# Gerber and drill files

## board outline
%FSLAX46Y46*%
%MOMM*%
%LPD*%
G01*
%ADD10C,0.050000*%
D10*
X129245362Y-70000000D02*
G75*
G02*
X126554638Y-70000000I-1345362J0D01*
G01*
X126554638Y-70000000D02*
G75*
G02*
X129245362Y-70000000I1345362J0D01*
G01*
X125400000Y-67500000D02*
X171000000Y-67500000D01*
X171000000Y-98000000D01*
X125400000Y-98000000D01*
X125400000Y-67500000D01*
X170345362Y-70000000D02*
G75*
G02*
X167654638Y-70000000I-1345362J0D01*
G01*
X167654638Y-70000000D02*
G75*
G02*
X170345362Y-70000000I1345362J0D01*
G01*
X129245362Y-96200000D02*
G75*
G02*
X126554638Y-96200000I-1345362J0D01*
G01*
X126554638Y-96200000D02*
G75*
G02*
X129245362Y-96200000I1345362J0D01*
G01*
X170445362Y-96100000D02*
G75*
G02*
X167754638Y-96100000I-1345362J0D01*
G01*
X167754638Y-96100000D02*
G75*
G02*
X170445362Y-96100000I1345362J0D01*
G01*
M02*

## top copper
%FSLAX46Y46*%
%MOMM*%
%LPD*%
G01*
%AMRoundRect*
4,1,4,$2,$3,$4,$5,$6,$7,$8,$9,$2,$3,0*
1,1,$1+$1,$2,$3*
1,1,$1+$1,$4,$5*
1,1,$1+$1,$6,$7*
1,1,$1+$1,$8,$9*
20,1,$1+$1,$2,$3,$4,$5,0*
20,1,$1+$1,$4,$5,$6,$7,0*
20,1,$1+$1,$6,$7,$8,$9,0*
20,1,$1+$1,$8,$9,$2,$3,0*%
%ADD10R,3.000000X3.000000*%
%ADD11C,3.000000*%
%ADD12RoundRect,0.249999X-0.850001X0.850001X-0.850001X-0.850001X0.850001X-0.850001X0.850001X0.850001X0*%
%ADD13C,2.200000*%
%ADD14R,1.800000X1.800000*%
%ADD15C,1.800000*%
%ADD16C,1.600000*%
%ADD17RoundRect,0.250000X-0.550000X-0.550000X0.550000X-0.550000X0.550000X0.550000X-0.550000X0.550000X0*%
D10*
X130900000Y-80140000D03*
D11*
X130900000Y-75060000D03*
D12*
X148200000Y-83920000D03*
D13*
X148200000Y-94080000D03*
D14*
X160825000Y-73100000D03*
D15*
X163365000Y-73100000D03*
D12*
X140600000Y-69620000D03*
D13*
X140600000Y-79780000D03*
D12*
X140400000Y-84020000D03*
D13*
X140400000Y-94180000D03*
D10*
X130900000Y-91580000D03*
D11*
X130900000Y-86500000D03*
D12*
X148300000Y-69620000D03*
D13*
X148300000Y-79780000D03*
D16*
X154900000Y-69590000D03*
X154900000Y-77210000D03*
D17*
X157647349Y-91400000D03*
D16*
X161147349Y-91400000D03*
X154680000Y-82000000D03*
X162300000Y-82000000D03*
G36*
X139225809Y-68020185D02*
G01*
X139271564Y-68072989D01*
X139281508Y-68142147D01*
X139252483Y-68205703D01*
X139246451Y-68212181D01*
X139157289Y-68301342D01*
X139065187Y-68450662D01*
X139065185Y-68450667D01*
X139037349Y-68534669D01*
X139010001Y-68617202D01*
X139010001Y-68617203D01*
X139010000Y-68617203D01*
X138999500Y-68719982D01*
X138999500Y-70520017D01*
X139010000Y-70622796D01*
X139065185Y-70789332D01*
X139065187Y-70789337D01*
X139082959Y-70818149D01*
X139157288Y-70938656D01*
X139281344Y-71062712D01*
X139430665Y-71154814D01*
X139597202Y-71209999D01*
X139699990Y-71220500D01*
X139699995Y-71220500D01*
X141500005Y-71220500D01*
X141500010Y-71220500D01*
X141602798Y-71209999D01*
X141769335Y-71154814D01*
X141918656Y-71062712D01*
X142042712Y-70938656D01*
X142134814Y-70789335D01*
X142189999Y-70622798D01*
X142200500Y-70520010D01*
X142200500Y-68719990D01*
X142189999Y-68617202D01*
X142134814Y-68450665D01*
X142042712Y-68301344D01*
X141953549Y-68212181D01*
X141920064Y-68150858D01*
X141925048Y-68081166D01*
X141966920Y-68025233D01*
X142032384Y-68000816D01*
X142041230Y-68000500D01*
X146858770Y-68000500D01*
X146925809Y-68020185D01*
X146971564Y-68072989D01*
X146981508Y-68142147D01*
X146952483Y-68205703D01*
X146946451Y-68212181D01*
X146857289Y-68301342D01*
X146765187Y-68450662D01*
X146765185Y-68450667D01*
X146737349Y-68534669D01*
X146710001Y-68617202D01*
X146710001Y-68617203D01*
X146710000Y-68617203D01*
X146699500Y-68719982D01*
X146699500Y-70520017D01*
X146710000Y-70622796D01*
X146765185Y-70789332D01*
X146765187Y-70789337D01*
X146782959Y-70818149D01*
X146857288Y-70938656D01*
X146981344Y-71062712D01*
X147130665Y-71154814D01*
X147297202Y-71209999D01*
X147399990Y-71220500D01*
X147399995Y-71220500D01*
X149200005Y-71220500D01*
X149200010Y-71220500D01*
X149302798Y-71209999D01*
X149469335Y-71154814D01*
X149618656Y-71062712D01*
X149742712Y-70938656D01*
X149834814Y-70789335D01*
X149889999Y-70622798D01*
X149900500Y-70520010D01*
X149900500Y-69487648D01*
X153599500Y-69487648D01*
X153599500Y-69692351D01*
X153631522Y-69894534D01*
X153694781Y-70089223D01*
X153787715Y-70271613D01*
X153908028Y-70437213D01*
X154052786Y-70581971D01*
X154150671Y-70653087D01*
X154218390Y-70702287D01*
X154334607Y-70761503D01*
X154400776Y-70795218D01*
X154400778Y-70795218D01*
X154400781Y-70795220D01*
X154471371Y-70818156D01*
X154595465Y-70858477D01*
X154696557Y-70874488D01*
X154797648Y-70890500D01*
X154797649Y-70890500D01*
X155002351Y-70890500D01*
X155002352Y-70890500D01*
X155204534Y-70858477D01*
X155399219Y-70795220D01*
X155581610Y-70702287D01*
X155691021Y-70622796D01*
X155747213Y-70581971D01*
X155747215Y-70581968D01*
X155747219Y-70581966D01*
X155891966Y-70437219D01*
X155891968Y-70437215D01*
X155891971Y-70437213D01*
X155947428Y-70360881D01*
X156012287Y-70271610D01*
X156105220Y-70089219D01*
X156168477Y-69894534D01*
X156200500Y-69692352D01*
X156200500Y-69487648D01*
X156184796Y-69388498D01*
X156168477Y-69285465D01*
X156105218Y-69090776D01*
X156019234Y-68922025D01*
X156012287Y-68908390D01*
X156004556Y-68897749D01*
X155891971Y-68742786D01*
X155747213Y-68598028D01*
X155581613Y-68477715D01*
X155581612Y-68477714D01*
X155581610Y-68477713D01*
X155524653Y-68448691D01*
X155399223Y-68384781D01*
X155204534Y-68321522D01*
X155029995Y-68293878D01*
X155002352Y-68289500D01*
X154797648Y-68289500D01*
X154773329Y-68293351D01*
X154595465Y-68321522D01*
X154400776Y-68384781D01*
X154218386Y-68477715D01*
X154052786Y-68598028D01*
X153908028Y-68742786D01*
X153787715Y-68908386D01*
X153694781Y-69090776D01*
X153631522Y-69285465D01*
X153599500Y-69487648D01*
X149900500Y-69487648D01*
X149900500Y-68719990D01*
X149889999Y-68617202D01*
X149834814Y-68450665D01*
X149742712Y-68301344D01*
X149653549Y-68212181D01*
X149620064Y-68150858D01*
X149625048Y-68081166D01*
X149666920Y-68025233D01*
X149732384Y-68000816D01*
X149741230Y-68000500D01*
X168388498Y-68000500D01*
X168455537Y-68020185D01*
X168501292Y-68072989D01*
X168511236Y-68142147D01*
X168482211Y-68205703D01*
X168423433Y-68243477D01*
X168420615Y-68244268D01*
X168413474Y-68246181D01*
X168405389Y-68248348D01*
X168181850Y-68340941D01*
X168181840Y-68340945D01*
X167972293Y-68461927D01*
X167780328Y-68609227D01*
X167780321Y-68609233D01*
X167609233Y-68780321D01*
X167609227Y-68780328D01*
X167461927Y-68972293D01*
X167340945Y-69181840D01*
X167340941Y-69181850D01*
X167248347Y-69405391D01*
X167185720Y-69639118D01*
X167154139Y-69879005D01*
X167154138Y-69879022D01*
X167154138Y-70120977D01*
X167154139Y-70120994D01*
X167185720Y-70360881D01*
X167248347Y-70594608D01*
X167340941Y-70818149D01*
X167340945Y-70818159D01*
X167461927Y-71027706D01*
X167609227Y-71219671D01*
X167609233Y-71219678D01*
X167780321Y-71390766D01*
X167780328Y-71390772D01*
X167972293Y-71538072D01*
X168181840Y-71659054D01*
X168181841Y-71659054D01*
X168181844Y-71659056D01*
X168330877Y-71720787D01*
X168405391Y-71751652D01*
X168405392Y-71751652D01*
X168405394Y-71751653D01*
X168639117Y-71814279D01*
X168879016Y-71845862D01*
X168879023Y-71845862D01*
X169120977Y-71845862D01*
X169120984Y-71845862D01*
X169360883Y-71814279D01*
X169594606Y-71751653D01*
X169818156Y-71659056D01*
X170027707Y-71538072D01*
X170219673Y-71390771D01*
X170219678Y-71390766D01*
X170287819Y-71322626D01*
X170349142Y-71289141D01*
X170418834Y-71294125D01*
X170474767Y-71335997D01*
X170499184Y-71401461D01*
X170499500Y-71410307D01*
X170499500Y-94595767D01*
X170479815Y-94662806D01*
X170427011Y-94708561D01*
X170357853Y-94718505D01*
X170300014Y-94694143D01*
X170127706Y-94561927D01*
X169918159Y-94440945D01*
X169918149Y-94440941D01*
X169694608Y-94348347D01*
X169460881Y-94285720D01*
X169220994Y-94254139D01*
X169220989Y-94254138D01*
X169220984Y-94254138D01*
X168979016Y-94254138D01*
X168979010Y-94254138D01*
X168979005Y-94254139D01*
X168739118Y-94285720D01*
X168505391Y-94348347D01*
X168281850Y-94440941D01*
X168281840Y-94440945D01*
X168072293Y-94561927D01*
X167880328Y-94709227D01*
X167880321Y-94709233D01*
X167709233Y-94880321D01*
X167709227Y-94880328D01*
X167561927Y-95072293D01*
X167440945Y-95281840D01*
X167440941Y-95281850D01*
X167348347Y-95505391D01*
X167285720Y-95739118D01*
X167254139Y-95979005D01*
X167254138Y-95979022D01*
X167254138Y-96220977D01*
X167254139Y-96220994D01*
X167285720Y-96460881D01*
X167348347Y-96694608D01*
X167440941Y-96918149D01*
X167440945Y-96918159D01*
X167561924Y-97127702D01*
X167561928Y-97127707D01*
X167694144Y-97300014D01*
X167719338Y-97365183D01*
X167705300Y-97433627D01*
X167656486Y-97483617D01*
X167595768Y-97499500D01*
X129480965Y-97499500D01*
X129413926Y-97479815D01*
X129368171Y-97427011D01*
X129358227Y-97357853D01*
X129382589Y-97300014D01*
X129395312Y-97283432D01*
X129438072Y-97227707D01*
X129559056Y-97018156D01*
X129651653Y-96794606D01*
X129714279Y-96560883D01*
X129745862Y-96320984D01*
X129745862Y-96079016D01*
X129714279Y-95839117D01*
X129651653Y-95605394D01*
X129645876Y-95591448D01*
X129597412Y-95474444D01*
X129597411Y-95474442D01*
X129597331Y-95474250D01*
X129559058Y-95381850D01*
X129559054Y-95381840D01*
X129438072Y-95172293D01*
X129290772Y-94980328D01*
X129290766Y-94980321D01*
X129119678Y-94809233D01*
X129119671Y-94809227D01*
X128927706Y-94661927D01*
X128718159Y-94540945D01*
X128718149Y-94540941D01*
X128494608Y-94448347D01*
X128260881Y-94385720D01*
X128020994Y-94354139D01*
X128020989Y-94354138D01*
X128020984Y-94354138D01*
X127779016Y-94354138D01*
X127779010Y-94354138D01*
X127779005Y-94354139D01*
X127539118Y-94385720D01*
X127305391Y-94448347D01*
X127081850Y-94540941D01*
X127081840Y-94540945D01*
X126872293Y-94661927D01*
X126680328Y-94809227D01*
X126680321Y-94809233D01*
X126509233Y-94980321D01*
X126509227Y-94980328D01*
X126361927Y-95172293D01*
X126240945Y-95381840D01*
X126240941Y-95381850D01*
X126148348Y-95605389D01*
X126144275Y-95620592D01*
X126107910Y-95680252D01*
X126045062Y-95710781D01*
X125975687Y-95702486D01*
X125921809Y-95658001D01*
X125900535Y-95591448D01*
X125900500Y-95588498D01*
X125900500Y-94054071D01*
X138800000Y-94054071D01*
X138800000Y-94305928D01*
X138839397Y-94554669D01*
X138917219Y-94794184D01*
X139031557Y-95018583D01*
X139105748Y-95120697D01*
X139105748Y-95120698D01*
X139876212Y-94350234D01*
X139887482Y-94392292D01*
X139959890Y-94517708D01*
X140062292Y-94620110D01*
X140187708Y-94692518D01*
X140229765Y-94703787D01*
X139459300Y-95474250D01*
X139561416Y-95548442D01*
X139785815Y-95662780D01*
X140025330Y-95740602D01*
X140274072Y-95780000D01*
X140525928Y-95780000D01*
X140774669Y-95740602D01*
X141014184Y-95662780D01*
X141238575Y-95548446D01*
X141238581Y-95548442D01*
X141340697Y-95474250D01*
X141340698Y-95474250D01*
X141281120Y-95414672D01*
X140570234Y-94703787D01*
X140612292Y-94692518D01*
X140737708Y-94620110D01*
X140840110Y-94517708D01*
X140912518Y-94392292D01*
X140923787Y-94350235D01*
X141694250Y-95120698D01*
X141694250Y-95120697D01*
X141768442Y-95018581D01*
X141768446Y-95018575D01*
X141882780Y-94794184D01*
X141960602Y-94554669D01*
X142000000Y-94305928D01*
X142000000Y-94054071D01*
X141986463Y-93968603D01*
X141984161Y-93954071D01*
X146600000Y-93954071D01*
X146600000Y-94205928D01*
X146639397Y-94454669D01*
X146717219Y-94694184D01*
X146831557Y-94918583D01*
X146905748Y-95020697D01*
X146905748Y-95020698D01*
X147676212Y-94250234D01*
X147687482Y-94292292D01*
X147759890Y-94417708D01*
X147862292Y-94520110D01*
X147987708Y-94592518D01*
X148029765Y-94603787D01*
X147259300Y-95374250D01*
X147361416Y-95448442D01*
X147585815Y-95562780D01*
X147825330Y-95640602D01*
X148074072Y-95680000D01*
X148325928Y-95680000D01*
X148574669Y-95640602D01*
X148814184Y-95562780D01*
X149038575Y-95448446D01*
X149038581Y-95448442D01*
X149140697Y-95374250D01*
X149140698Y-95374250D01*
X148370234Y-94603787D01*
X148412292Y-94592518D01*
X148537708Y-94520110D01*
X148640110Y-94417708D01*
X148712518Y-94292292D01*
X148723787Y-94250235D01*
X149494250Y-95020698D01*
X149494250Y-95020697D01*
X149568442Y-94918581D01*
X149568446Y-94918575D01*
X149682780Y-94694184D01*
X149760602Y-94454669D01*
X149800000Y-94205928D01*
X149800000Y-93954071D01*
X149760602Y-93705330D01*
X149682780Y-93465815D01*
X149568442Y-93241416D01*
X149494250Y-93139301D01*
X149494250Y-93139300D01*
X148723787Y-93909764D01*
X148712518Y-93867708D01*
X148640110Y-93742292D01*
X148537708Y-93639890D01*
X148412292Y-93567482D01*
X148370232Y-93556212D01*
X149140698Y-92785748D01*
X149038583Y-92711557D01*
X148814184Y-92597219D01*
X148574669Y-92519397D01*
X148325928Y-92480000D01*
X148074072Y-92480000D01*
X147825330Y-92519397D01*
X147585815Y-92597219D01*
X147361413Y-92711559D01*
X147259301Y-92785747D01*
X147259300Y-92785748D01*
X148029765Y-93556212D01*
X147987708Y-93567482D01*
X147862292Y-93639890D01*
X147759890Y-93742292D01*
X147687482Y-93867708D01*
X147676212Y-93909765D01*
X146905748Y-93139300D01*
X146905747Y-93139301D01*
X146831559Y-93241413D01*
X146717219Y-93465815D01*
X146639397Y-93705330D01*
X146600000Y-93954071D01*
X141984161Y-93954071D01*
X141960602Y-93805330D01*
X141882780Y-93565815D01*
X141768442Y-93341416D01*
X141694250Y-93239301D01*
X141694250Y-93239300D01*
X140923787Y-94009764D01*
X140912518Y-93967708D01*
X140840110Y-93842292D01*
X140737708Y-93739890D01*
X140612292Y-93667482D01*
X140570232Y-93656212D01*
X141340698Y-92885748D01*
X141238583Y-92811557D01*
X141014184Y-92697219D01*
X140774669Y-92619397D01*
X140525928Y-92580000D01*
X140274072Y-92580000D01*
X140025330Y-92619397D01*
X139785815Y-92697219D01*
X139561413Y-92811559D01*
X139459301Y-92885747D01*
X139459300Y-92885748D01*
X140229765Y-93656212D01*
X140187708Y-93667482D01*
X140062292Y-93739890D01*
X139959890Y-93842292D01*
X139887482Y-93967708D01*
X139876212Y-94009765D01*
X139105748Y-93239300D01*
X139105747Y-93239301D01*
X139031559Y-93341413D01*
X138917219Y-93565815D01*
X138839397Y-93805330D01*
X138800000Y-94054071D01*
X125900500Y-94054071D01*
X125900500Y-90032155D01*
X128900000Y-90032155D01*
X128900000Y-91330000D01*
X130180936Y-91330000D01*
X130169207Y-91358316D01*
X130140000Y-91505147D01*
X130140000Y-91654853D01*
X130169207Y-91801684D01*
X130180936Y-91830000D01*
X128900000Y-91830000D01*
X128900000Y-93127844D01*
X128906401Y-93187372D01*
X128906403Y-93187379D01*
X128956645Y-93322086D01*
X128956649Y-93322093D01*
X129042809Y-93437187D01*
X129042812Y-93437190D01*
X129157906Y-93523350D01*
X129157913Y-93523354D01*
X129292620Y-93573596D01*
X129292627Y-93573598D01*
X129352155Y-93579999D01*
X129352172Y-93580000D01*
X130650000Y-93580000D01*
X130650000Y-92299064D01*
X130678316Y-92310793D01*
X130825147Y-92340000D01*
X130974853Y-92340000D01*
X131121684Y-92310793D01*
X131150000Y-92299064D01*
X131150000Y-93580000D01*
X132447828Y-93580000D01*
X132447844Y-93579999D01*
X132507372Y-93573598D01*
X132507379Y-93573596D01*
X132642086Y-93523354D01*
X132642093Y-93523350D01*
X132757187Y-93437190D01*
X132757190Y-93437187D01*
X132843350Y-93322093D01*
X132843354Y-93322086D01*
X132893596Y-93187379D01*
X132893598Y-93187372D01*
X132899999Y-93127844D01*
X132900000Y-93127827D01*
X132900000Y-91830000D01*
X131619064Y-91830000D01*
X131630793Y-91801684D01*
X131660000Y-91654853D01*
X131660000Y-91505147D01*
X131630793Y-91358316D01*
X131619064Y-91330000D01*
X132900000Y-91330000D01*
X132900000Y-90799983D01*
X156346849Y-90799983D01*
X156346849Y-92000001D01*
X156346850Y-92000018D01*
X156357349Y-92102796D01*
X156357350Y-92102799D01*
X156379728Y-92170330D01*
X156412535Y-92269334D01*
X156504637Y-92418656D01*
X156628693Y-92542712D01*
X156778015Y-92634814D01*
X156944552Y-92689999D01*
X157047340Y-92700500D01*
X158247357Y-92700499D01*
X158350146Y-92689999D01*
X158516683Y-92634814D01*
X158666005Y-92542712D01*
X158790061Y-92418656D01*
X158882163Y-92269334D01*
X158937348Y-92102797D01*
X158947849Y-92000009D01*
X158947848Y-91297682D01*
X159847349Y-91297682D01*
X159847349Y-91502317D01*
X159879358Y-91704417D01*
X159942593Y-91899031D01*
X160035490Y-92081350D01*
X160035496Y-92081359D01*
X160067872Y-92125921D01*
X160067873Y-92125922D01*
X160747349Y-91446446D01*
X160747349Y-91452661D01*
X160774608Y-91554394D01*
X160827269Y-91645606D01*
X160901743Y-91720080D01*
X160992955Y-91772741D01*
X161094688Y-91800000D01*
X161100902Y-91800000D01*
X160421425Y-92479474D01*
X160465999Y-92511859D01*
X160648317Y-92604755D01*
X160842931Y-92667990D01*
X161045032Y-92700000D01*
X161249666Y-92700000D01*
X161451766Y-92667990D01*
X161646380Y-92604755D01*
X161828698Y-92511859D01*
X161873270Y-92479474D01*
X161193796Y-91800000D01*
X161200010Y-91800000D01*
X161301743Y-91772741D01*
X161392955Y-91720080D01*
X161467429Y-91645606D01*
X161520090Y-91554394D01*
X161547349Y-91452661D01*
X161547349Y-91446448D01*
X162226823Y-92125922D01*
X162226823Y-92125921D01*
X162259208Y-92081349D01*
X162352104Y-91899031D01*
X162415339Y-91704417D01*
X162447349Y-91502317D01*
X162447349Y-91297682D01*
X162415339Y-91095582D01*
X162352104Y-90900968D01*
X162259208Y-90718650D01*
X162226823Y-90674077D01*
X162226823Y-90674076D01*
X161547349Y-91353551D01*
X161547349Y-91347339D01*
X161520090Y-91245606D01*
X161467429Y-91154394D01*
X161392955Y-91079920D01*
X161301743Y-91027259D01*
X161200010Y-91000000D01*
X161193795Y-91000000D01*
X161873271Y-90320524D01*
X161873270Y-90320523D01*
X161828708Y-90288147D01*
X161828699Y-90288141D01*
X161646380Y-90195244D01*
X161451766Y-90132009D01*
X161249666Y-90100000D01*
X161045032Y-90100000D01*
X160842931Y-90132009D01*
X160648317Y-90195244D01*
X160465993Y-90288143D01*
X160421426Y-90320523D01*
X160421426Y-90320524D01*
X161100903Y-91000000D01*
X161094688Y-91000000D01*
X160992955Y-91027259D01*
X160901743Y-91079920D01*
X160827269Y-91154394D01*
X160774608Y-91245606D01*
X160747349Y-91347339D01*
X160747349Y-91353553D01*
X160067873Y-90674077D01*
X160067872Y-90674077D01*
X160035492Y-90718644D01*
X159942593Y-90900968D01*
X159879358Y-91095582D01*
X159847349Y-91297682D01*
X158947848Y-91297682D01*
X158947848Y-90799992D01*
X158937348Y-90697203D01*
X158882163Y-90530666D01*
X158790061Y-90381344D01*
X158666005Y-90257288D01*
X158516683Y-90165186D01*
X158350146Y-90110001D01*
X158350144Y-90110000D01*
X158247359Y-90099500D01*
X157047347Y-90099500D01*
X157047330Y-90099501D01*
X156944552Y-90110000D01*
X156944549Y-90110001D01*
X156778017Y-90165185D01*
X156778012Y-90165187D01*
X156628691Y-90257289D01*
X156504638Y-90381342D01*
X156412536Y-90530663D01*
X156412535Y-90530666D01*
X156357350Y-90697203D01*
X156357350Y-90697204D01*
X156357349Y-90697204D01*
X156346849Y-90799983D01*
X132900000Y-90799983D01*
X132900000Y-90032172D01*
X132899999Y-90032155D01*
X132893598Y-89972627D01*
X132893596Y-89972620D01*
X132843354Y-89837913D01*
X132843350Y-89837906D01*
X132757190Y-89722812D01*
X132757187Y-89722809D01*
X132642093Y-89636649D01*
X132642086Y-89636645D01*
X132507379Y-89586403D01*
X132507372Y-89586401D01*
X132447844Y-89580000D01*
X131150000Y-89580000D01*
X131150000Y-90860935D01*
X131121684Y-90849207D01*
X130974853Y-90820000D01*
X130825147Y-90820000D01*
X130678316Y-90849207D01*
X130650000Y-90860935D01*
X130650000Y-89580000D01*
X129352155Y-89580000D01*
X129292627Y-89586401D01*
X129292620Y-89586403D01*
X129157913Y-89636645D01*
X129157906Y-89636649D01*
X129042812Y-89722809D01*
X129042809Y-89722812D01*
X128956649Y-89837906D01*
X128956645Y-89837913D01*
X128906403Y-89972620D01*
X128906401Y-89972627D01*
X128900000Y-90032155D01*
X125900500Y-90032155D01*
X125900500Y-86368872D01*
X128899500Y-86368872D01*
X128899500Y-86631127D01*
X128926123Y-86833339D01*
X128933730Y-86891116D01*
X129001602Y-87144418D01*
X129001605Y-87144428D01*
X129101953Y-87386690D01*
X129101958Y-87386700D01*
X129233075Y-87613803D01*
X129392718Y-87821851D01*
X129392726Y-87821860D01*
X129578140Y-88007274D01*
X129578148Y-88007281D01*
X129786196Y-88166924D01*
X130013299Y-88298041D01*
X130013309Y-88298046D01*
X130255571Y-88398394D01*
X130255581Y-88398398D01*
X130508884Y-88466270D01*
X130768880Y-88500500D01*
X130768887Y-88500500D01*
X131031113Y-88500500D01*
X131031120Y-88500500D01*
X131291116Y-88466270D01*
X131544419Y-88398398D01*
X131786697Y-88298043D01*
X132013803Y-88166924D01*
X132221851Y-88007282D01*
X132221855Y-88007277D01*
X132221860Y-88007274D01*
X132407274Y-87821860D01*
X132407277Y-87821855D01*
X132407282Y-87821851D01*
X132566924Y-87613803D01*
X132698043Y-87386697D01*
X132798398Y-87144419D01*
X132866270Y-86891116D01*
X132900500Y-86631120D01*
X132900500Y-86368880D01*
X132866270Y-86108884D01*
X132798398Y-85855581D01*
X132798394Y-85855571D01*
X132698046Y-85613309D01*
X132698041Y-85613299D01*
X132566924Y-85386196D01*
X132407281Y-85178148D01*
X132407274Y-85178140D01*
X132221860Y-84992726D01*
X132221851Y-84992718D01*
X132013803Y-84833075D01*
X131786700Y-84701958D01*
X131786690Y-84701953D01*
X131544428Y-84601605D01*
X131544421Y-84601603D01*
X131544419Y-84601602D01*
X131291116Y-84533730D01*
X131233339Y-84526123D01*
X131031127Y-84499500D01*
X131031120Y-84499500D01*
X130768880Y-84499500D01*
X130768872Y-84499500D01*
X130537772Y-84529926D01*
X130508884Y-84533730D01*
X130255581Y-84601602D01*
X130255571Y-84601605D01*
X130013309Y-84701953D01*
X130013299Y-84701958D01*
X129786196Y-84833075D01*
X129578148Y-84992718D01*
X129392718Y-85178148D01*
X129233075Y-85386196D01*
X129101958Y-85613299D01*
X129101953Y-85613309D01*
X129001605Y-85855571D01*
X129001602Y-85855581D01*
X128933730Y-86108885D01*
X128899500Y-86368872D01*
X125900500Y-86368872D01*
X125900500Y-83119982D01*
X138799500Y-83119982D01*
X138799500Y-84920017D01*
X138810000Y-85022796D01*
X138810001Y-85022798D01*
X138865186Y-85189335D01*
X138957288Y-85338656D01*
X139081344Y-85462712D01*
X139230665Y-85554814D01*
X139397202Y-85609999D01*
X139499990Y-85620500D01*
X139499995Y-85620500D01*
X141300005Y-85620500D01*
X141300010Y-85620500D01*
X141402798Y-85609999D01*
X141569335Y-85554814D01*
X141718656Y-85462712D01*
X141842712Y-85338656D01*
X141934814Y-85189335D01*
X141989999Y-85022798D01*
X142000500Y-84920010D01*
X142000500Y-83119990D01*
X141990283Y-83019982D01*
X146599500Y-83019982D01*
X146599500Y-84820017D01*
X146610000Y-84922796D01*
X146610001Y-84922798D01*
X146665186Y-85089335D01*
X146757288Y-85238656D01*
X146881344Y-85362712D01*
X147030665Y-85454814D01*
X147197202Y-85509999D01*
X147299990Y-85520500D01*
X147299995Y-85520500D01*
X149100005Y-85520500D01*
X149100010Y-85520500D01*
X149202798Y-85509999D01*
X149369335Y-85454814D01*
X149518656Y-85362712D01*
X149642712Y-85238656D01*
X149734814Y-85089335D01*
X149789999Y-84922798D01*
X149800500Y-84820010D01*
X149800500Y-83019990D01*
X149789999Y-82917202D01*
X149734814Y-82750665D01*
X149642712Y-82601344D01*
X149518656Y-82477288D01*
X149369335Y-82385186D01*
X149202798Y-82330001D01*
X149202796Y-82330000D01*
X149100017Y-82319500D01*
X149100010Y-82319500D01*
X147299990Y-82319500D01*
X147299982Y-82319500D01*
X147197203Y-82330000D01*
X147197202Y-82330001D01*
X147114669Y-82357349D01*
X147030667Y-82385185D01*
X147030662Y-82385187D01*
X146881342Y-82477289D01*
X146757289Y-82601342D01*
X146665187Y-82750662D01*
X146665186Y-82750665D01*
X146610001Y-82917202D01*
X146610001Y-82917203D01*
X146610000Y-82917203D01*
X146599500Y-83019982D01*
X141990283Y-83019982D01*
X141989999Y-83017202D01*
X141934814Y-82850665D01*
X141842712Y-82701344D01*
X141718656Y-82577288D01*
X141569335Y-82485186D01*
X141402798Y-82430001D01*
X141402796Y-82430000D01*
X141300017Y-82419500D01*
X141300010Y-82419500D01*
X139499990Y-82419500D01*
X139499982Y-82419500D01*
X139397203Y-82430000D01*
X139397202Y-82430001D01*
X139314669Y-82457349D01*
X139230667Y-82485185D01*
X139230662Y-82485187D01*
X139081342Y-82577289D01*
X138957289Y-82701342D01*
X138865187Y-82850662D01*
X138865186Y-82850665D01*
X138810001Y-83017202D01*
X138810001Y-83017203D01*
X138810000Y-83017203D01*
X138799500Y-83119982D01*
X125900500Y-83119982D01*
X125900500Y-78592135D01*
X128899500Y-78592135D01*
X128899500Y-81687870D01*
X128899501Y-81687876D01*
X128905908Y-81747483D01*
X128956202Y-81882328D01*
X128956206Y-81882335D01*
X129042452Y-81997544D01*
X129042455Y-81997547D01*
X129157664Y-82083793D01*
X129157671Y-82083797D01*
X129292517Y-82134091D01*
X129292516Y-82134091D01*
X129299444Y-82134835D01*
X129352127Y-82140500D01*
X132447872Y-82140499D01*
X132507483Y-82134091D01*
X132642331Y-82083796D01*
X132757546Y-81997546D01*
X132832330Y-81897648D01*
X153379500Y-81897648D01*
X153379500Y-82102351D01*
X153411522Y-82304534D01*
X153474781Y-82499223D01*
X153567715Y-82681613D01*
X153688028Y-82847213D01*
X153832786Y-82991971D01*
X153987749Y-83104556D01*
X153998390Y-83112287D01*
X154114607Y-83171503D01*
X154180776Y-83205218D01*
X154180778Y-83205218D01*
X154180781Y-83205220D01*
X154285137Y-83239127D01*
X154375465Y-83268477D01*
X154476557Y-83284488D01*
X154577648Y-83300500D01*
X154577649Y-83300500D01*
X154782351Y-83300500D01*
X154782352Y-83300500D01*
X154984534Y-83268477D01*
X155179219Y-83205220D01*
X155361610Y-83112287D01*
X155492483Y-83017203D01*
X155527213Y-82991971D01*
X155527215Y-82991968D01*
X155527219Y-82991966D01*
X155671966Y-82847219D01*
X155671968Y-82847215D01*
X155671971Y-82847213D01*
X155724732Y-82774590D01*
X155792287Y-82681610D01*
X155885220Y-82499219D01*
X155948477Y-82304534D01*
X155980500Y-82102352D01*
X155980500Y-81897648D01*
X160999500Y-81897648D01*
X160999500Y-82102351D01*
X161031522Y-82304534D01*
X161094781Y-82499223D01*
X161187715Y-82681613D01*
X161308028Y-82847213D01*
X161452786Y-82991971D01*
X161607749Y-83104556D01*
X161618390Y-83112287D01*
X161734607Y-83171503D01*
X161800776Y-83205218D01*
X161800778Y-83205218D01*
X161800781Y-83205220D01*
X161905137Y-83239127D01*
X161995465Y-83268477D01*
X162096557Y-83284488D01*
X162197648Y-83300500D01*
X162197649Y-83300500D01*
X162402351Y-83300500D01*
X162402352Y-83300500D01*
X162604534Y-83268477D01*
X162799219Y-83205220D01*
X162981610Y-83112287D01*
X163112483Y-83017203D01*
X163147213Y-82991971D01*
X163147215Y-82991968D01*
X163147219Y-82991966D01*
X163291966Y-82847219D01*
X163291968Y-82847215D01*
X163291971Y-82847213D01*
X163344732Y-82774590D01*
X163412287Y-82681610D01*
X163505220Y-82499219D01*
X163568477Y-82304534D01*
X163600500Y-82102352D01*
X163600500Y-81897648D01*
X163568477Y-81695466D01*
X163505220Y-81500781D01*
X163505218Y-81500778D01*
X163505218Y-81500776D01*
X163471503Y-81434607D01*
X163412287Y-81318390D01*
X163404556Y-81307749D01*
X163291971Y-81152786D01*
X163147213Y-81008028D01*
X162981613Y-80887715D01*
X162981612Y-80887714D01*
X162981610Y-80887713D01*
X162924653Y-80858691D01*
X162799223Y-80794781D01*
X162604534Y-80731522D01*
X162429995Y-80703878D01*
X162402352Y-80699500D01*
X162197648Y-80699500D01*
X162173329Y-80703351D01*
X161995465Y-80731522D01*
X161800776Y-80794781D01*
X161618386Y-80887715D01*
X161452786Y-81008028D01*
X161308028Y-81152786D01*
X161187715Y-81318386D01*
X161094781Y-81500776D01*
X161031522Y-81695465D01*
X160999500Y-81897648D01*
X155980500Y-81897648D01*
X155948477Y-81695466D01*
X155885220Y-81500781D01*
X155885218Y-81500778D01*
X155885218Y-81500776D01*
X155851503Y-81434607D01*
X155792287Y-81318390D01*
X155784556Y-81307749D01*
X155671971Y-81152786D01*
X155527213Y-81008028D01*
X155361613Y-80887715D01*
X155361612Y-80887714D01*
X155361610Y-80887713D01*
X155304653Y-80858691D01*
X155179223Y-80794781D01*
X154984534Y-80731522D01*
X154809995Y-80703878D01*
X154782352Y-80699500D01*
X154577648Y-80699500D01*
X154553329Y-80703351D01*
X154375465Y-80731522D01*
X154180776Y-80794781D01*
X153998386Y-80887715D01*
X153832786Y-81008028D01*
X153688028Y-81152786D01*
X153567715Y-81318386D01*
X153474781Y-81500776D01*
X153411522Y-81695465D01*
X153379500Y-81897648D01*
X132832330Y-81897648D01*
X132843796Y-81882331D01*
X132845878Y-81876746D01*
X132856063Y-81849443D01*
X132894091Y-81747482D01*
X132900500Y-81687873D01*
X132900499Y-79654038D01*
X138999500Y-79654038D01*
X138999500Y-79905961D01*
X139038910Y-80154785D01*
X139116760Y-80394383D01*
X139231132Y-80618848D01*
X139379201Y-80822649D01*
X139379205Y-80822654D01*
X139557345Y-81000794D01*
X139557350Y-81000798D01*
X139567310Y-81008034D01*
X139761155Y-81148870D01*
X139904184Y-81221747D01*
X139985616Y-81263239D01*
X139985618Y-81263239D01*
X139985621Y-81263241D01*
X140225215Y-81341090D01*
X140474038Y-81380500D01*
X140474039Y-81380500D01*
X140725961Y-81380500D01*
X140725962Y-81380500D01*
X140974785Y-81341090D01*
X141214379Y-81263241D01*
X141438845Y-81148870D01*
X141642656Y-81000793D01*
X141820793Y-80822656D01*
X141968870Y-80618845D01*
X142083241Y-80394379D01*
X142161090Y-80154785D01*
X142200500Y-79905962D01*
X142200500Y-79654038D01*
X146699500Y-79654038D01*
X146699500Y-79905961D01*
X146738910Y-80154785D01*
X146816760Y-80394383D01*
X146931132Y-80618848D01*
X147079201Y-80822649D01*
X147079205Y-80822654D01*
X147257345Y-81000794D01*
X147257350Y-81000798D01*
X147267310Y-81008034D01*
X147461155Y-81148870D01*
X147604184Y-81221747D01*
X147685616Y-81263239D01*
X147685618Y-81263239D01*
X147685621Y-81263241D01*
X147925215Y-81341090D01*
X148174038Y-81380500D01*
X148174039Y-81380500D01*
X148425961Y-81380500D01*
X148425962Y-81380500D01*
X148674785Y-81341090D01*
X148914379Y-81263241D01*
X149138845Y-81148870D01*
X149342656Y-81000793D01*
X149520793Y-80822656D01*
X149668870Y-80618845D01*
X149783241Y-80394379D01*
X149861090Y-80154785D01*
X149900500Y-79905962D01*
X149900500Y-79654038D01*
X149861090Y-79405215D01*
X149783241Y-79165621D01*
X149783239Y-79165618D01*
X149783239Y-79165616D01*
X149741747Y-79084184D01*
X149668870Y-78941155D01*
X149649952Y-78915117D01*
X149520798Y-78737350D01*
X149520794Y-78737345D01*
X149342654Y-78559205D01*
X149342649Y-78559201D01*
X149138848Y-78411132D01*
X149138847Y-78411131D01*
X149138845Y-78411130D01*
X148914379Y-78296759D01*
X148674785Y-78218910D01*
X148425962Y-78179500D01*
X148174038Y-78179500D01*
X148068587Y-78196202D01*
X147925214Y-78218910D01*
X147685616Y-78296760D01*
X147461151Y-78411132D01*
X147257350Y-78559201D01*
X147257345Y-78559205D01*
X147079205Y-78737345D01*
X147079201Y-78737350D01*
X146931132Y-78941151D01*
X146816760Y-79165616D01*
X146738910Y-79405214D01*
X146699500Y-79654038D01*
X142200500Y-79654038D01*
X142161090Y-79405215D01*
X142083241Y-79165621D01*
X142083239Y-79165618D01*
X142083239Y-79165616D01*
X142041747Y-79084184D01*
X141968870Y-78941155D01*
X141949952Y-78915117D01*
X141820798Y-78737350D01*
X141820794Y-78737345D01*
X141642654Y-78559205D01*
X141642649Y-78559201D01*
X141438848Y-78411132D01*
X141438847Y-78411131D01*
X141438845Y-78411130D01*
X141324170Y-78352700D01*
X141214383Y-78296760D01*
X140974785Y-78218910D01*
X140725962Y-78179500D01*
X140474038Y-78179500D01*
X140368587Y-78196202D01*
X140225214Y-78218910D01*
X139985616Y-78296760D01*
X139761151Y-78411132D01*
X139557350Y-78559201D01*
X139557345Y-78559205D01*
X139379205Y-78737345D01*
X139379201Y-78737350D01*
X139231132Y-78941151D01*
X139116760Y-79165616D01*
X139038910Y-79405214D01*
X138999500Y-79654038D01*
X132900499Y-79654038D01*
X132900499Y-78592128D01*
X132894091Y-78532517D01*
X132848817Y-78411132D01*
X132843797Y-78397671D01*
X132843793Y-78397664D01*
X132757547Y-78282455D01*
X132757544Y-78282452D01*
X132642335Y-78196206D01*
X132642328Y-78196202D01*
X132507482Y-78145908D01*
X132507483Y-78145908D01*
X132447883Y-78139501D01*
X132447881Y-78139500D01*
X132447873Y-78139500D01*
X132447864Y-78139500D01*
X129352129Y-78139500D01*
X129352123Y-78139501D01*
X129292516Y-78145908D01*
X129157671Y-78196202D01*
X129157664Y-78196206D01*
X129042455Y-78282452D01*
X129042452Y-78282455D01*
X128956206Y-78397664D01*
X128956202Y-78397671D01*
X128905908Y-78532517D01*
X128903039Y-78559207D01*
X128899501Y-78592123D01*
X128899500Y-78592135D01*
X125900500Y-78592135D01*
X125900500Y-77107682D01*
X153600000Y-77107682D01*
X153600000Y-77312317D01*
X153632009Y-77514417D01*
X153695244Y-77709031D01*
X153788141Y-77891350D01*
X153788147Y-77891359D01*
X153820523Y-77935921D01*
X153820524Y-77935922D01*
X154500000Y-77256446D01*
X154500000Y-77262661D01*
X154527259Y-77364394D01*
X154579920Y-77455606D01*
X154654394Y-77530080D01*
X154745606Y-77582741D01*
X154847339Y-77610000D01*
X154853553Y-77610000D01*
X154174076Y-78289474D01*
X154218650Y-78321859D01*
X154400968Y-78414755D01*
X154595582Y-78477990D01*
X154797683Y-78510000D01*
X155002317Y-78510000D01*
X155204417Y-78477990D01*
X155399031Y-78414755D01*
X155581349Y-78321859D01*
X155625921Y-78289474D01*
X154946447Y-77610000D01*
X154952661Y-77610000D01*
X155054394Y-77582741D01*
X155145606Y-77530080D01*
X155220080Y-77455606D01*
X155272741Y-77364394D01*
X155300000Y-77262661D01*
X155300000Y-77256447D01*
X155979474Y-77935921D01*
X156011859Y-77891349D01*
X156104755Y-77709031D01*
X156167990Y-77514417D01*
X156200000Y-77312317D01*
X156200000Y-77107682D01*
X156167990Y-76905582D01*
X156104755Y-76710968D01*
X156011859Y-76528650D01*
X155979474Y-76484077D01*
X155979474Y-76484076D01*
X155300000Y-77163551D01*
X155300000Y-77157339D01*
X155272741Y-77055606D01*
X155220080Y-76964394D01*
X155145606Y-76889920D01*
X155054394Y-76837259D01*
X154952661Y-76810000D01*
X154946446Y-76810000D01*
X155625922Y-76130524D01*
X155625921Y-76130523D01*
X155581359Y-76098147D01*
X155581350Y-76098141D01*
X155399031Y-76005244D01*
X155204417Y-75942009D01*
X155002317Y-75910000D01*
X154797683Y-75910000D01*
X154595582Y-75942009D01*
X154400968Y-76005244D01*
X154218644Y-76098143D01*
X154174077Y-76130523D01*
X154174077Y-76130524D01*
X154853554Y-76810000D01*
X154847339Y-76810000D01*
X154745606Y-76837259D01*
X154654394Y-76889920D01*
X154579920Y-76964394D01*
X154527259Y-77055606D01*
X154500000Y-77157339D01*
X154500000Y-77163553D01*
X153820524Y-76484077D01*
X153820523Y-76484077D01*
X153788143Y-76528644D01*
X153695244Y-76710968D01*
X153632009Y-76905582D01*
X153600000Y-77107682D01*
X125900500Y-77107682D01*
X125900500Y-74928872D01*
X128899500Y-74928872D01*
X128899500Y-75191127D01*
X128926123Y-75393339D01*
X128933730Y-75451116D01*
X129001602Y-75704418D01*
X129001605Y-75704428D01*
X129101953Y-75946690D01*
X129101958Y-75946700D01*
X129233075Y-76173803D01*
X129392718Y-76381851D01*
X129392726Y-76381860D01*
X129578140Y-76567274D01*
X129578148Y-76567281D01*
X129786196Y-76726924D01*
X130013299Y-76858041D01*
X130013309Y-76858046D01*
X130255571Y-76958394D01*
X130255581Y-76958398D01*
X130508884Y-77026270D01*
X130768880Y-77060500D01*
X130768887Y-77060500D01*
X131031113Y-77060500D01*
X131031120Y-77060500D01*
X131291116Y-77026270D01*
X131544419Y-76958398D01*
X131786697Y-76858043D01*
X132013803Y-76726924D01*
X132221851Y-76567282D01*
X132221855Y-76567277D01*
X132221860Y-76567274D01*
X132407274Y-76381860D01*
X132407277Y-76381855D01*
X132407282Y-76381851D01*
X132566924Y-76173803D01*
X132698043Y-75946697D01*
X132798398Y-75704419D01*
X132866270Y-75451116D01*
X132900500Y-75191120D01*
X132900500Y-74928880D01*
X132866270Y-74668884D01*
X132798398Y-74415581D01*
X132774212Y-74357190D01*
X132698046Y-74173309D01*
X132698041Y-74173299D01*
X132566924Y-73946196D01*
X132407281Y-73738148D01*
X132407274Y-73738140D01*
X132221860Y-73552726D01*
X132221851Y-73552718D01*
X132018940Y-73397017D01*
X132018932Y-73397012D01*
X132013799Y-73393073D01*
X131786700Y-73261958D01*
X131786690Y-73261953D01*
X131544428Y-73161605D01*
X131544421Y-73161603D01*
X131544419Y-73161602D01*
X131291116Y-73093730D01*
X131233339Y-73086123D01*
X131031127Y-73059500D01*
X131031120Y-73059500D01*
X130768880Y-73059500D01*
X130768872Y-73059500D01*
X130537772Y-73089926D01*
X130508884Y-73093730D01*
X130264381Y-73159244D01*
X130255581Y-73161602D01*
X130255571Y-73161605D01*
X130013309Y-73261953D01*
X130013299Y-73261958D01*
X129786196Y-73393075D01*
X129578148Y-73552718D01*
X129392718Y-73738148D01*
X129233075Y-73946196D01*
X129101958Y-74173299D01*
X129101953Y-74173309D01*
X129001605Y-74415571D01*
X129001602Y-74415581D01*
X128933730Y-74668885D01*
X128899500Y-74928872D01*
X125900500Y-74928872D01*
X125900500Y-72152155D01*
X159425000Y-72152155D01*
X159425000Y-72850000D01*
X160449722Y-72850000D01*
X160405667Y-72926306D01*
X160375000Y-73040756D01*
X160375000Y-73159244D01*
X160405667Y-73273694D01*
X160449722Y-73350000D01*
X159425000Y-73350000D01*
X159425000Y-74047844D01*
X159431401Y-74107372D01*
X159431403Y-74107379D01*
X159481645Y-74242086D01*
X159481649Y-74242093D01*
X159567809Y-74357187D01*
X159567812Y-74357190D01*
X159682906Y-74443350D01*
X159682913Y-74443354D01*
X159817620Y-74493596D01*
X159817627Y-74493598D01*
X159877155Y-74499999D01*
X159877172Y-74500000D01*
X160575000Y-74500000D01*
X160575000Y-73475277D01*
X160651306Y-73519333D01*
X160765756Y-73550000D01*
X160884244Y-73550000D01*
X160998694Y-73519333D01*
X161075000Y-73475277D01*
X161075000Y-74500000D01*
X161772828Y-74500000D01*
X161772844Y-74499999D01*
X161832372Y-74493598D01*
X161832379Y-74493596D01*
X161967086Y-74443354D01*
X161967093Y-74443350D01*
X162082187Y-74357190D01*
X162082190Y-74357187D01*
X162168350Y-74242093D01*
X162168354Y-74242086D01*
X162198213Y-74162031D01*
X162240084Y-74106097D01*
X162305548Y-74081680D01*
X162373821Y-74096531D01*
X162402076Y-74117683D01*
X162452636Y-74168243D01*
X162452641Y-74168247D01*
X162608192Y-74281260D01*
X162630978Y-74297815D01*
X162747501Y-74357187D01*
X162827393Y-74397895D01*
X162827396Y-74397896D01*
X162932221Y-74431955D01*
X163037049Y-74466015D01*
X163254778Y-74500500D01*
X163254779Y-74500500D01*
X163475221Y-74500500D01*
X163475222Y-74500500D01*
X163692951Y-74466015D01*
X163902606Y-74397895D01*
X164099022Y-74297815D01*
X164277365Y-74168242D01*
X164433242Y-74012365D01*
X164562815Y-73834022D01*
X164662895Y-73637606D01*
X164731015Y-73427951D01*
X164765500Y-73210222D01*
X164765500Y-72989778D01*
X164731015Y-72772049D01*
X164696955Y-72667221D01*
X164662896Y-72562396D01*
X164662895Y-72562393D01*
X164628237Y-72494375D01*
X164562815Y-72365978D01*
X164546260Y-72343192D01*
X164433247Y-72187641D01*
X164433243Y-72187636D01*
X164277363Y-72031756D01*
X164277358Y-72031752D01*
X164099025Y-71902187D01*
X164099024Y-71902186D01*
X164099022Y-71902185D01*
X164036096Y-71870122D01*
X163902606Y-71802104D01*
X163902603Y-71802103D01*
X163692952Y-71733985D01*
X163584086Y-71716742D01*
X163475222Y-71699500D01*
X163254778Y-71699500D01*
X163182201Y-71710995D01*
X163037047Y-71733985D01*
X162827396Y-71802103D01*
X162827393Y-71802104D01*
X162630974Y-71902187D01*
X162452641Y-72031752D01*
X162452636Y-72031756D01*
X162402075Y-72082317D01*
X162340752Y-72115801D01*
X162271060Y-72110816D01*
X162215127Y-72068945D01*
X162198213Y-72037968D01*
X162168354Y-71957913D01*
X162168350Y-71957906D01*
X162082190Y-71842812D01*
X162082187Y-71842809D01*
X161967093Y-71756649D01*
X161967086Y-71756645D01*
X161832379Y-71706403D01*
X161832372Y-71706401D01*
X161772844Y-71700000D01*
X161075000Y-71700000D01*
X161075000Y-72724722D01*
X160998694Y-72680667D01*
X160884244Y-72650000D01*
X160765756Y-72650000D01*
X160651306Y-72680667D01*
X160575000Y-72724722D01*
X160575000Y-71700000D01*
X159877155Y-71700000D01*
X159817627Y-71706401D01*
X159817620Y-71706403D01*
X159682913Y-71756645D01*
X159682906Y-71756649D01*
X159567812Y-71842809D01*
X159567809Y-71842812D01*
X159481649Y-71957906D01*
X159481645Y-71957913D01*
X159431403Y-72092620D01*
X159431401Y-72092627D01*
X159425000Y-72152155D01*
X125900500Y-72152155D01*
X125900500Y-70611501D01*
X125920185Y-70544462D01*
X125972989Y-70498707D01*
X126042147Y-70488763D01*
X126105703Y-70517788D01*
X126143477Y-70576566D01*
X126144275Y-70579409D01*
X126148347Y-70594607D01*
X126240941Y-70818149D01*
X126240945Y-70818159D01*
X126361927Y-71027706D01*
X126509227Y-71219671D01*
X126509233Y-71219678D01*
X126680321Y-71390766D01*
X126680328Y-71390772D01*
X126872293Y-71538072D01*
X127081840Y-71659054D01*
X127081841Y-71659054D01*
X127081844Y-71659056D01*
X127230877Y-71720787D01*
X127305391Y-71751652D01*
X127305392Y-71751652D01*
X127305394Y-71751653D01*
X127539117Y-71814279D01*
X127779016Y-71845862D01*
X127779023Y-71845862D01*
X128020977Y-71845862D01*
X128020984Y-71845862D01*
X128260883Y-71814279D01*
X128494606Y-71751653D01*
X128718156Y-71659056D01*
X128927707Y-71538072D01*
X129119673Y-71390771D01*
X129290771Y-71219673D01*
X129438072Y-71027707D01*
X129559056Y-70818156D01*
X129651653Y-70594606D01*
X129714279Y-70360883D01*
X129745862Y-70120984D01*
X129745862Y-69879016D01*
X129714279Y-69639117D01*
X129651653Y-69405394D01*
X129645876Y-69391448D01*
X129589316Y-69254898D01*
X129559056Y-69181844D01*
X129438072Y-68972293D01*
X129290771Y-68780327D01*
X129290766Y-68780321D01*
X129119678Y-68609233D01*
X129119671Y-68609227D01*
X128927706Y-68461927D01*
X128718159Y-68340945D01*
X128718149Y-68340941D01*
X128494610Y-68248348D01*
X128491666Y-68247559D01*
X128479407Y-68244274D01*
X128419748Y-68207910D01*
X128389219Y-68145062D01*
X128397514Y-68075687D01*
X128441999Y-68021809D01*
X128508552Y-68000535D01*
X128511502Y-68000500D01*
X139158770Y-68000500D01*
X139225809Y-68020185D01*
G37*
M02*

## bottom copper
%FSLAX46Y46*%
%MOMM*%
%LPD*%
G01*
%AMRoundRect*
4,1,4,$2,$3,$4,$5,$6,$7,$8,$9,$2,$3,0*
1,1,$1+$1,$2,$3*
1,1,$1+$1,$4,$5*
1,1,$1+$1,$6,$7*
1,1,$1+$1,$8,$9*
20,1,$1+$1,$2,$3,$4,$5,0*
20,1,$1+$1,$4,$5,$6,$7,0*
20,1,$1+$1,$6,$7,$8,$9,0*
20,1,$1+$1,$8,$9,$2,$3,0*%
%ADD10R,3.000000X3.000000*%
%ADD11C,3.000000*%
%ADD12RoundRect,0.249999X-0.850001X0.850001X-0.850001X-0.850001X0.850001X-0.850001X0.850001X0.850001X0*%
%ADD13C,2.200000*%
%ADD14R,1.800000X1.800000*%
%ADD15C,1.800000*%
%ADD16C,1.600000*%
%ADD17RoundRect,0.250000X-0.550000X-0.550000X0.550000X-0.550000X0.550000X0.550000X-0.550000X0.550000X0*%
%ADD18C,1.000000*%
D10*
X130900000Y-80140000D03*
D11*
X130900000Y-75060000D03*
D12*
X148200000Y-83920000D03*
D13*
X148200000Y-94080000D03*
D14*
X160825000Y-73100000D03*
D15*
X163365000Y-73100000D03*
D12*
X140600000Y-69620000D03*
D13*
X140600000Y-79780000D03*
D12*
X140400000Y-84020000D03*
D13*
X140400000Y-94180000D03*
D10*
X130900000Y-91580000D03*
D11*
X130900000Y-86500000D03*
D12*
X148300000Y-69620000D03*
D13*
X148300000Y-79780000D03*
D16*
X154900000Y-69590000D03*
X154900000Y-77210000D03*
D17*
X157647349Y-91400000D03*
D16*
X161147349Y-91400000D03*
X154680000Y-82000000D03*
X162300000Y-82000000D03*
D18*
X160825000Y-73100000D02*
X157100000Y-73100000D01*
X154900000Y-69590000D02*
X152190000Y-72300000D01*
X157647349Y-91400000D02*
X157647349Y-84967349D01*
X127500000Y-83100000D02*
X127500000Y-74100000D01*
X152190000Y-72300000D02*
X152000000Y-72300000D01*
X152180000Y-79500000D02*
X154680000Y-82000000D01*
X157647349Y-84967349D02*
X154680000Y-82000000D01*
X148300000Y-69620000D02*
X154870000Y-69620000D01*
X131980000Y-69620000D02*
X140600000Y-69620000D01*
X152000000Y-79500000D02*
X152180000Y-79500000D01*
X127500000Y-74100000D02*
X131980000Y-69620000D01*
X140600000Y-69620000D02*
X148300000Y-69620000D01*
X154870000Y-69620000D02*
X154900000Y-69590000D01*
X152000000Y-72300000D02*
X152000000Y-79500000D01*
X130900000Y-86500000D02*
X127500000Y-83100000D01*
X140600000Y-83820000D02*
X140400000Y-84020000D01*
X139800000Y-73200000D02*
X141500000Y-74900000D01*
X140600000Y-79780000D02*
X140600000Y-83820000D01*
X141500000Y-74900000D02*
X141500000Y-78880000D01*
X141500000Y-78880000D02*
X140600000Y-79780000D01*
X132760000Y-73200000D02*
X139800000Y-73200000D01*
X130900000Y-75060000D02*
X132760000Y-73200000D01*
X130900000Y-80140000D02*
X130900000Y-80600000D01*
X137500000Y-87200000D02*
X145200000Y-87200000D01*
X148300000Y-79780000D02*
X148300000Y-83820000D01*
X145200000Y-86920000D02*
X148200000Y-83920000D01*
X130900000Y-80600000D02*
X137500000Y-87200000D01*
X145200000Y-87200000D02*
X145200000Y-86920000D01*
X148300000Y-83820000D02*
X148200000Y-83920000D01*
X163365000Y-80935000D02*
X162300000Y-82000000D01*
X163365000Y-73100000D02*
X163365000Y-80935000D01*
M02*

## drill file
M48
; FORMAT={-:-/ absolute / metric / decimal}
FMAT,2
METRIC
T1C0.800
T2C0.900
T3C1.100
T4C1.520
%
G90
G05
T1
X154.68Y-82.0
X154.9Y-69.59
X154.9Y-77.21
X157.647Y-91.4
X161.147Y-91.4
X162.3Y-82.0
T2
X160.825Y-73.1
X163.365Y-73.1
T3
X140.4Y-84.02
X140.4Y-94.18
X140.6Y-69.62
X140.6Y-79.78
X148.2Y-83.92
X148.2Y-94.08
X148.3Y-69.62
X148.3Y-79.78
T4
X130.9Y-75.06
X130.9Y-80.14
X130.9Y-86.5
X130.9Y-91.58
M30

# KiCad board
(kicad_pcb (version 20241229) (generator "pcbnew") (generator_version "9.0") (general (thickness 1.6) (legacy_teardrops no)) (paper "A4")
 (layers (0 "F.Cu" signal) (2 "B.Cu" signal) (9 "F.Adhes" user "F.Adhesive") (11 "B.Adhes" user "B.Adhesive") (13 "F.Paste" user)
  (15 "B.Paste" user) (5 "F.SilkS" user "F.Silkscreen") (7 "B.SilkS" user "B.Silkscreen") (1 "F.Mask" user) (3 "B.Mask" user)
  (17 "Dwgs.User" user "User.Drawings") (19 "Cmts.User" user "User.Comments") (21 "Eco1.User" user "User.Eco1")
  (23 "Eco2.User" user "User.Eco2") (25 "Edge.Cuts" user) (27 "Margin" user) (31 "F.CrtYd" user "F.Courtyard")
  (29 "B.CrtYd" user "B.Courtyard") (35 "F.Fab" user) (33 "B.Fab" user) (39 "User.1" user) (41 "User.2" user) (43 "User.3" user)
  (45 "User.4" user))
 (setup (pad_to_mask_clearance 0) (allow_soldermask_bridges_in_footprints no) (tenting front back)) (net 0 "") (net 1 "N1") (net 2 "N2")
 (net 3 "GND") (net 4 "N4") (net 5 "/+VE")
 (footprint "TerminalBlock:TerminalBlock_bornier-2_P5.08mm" (layer "F.Cu") (at 130.9 80.14 90)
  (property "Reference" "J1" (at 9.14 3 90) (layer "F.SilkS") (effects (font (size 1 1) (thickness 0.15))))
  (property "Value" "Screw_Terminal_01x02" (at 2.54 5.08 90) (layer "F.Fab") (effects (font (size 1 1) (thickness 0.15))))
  (pad "1" thru_hole rect (at 0 0 90) (size 3 3) (drill 1.52) (layers "*.Cu" "*.Mask") (remove_unused_layers no) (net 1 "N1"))
  (pad "2" thru_hole circle (at 5.08 0 90) (size 3 3) (drill 1.52) (layers "*.Cu" "*.Mask") (remove_unused_layers no) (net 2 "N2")))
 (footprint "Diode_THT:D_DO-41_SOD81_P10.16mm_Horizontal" (layer "F.Cu") (at 148.2 83.92 -90)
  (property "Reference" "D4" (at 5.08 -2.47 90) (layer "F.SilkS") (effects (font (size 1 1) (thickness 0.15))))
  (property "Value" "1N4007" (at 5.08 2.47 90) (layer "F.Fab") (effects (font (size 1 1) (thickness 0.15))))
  (pad "1" thru_hole roundrect (at 0 0 270) (size 2.2 2.2) (drill 1.1) (layers "*.Cu" "*.Mask") (remove_unused_layers no)
   (roundrect_rratio 0.113636) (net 1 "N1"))
  (pad "2" thru_hole circle (at 10.16 0 270) (size 2.2 2.2) (drill 1.1) (layers "*.Cu" "*.Mask") (remove_unused_layers no) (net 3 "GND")))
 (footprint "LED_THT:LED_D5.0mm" (layer "F.Cu") (at 160.825 73.1)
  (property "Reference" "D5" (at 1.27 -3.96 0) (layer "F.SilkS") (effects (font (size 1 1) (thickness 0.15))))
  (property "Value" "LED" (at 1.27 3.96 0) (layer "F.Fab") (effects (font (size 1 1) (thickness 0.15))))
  (pad "1" thru_hole rect (at 0 0) (size 1.8 1.8) (drill 0.9) (layers "*.Cu" "*.Mask") (remove_unused_layers no) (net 3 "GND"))
  (pad "2" thru_hole circle (at 2.54 0) (size 1.8 1.8) (drill 0.9) (layers "*.Cu" "*.Mask") (remove_unused_layers no) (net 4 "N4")))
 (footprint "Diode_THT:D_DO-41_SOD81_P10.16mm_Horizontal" (layer "F.Cu") (at 140.6 69.62 -90)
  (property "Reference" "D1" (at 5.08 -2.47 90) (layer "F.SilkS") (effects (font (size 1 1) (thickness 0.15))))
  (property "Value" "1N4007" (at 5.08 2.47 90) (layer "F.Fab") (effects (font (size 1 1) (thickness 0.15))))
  (pad "1" thru_hole roundrect (at 0 0 270) (size 2.2 2.2) (drill 1.1) (layers "*.Cu" "*.Mask") (remove_unused_layers no)
   (roundrect_rratio 0.113636) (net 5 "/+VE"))
  (pad "2" thru_hole circle (at 10.16 0 270) (size 2.2 2.2) (drill 1.1) (layers "*.Cu" "*.Mask") (remove_unused_layers no) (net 2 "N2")))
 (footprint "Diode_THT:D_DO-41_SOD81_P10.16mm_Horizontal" (layer "F.Cu") (at 140.4 84.02 -90)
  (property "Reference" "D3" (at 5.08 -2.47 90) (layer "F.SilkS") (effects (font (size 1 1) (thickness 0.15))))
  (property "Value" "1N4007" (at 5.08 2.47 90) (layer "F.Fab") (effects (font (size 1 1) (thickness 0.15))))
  (pad "1" thru_hole roundrect (at 0 0 270) (size 2.2 2.2) (drill 1.1) (layers "*.Cu" "*.Mask") (remove_unused_layers no)
   (roundrect_rratio 0.113636) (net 2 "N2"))
  (pad "2" thru_hole circle (at 10.16 0 270) (size 2.2 2.2) (drill 1.1) (layers "*.Cu" "*.Mask") (remove_unused_layers no) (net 3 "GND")))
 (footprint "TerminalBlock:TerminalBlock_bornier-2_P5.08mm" (layer "F.Cu") (at 130.9 91.58 90)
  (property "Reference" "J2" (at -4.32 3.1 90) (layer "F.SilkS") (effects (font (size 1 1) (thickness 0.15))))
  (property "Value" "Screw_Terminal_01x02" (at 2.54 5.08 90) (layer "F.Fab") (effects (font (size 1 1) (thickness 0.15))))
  (pad "1" thru_hole rect (at 0 0 90) (size 3 3) (drill 1.52) (layers "*.Cu" "*.Mask") (remove_unused_layers no) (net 3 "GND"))
  (pad "2" thru_hole circle (at 5.08 0 90) (size 3 3) (drill 1.52) (layers "*.Cu" "*.Mask") (remove_unused_layers no) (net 5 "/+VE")))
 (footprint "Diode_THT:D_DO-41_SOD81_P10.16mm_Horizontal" (layer "F.Cu") (at 148.3 69.62 -90)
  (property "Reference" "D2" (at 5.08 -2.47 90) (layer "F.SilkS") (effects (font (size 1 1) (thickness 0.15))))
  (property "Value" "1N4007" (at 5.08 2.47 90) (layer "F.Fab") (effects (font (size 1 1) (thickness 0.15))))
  (pad "1" thru_hole roundrect (at 0 0 270) (size 2.2 2.2) (drill 1.1) (layers "*.Cu" "*.Mask") (remove_unused_layers no)
   (roundrect_rratio 0.113636) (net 5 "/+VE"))
  (pad "2" thru_hole circle (at 10.16 0 270) (size 2.2 2.2) (drill 1.1) (layers "*.Cu" "*.Mask") (remove_unused_layers no) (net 1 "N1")))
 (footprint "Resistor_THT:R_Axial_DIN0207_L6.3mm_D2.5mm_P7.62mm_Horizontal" (layer "F.Cu") (at 154.9 69.59 -90)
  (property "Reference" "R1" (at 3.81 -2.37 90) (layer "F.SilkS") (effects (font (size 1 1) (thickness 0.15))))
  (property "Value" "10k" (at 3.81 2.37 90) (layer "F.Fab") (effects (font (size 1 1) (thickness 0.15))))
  (pad "1" thru_hole circle (at 0 0 270) (size 1.6 1.6) (drill 0.8) (layers "*.Cu" "*.Mask") (remove_unused_layers no) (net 5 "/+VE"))
  (pad "2" thru_hole circle (at 7.62 0 270) (size 1.6 1.6) (drill 0.8) (layers "*.Cu" "*.Mask") (remove_unused_layers no) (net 3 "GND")))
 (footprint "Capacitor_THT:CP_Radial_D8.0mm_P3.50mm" (layer "F.Cu") (at 157.647349 91.4)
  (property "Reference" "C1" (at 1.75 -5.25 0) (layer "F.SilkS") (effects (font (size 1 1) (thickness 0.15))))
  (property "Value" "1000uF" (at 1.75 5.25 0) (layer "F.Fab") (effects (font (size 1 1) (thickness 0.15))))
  (pad "1" thru_hole roundrect (at 0 0) (size 1.6 1.6) (drill 0.8) (layers "*.Cu" "*.Mask") (remove_unused_layers no)
   (roundrect_rratio 0.15625) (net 5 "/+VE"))
  (pad "2" thru_hole circle (at 3.5 0) (size 1.6 1.6) (drill 0.8) (layers "*.Cu" "*.Mask") (remove_unused_layers no) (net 3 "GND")))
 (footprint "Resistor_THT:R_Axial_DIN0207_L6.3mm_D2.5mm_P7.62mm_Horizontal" (layer "F.Cu") (at 154.68 82)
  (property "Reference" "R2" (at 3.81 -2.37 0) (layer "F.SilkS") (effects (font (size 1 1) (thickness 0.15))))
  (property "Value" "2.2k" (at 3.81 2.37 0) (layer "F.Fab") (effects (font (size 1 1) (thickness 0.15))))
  (pad "1" thru_hole circle (at 0 0) (size 1.6 1.6) (drill 0.8) (layers "*.Cu" "*.Mask") (remove_unused_layers no) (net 5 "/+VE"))
  (pad "2" thru_hole circle (at 7.62 0) (size 1.6 1.6) (drill 0.8) (layers "*.Cu" "*.Mask") (remove_unused_layers no) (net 4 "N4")))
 (gr_circle (center 127.9 70) (end 129.245362 70) (stroke (width 0.05) (type default)) (fill no) (layer "Edge.Cuts"))
 (gr_rect (start 125.4 67.5) (end 171 98) (stroke (width 0.05) (type default)) (fill no) (layer "Edge.Cuts"))
 (gr_circle (center 169 70) (end 170.345362 70) (stroke (width 0.05) (type default)) (fill no) (layer "Edge.Cuts"))
 (gr_circle (center 127.9 96.2) (end 129.245362 96.2) (stroke (width 0.05) (type default)) (fill no) (layer "Edge.Cuts"))
 (gr_circle (center 169.1 96.1) (end 170.445362 96.1) (stroke (width 0.05) (type default)) (fill no) (layer "Edge.Cuts"))
 (segment (start 160.825 73.1) (end 157.1 73.1) (width 1) (layer "B.Cu") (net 3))
 (segment (start 154.9 69.59) (end 152.19 72.3) (width 1) (layer "B.Cu") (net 5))
 (segment (start 157.647349 91.4) (end 157.647349 84.967349) (width 1) (layer "B.Cu") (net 5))
 (segment (start 127.5 83.1) (end 127.5 74.1) (width 1) (layer "B.Cu") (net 5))
 (segment (start 152.19 72.3) (end 152 72.3) (width 1) (layer "B.Cu") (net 5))
 (segment (start 152.18 79.5) (end 154.68 82) (width 1) (layer "B.Cu") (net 5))
 (segment (start 157.647349 84.967349) (end 154.68 82) (width 1) (layer "B.Cu") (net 5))
 (segment (start 148.3 69.62) (end 154.87 69.62) (width 1) (layer "B.Cu") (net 5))
 (segment (start 131.98 69.62) (end 140.6 69.62) (width 1) (layer "B.Cu") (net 5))
 (segment (start 152 79.5) (end 152.18 79.5) (width 1) (layer "B.Cu") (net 5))
 (segment (start 127.5 74.1) (end 131.98 69.62) (width 1) (layer "B.Cu") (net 5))
 (segment (start 140.6 69.62) (end 148.3 69.62) (width 1) (layer "B.Cu") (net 5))
 (segment (start 154.87 69.62) (end 154.9 69.59) (width 1) (layer "B.Cu") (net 5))
 (segment (start 152 72.3) (end 152 79.5) (width 1) (layer "B.Cu") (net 5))
 (segment (start 130.9 86.5) (end 127.5 83.1) (width 1) (layer "B.Cu") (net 5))
 (segment (start 140.6 83.82) (end 140.4 84.02) (width 1) (layer "B.Cu") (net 2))
 (segment (start 139.8 73.2) (end 141.5 74.9) (width 1) (layer "B.Cu") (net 2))
 (segment (start 140.6 79.78) (end 140.6 83.82) (width 1) (layer "B.Cu") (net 2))
 (segment (start 141.5 74.9) (end 141.5 78.88) (width 1) (layer "B.Cu") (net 2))
 (segment (start 141.5 78.88) (end 140.6 79.78) (width 1) (layer "B.Cu") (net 2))
 (segment (start 132.76 73.2) (end 139.8 73.2) (width 1) (layer "B.Cu") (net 2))
 (segment (start 130.9 75.06) (end 132.76 73.2) (width 1) (layer "B.Cu") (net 2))
 (segment (start 130.9 80.14) (end 130.9 80.6) (width 1) (layer "B.Cu") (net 1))
 (segment (start 137.5 87.2) (end 145.2 87.2) (width 1) (layer "B.Cu") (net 1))
 (segment (start 148.3 79.78) (end 148.3 83.82) (width 1) (layer "B.Cu") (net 1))
 (segment (start 145.2 86.92) (end 148.2 83.92) (width 1) (layer "B.Cu") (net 1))
 (segment (start 130.9 80.6) (end 137.5 87.2) (width 1) (layer "B.Cu") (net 1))
 (segment (start 145.2 87.2) (end 145.2 86.92) (width 1) (layer "B.Cu") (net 1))
 (segment (start 148.3 83.82) (end 148.2 83.92) (width 1) (layer "B.Cu") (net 1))
 (segment (start 163.365 80.935) (end 162.3 82) (width 1) (layer "B.Cu") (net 4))
 (segment (start 163.365 73.1) (end 163.365 80.935) (width 1) (layer "B.Cu") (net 4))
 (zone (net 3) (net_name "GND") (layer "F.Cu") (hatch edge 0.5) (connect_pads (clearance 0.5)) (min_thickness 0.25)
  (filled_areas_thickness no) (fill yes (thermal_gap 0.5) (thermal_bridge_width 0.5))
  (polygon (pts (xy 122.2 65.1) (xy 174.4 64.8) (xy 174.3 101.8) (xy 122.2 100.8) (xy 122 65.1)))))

